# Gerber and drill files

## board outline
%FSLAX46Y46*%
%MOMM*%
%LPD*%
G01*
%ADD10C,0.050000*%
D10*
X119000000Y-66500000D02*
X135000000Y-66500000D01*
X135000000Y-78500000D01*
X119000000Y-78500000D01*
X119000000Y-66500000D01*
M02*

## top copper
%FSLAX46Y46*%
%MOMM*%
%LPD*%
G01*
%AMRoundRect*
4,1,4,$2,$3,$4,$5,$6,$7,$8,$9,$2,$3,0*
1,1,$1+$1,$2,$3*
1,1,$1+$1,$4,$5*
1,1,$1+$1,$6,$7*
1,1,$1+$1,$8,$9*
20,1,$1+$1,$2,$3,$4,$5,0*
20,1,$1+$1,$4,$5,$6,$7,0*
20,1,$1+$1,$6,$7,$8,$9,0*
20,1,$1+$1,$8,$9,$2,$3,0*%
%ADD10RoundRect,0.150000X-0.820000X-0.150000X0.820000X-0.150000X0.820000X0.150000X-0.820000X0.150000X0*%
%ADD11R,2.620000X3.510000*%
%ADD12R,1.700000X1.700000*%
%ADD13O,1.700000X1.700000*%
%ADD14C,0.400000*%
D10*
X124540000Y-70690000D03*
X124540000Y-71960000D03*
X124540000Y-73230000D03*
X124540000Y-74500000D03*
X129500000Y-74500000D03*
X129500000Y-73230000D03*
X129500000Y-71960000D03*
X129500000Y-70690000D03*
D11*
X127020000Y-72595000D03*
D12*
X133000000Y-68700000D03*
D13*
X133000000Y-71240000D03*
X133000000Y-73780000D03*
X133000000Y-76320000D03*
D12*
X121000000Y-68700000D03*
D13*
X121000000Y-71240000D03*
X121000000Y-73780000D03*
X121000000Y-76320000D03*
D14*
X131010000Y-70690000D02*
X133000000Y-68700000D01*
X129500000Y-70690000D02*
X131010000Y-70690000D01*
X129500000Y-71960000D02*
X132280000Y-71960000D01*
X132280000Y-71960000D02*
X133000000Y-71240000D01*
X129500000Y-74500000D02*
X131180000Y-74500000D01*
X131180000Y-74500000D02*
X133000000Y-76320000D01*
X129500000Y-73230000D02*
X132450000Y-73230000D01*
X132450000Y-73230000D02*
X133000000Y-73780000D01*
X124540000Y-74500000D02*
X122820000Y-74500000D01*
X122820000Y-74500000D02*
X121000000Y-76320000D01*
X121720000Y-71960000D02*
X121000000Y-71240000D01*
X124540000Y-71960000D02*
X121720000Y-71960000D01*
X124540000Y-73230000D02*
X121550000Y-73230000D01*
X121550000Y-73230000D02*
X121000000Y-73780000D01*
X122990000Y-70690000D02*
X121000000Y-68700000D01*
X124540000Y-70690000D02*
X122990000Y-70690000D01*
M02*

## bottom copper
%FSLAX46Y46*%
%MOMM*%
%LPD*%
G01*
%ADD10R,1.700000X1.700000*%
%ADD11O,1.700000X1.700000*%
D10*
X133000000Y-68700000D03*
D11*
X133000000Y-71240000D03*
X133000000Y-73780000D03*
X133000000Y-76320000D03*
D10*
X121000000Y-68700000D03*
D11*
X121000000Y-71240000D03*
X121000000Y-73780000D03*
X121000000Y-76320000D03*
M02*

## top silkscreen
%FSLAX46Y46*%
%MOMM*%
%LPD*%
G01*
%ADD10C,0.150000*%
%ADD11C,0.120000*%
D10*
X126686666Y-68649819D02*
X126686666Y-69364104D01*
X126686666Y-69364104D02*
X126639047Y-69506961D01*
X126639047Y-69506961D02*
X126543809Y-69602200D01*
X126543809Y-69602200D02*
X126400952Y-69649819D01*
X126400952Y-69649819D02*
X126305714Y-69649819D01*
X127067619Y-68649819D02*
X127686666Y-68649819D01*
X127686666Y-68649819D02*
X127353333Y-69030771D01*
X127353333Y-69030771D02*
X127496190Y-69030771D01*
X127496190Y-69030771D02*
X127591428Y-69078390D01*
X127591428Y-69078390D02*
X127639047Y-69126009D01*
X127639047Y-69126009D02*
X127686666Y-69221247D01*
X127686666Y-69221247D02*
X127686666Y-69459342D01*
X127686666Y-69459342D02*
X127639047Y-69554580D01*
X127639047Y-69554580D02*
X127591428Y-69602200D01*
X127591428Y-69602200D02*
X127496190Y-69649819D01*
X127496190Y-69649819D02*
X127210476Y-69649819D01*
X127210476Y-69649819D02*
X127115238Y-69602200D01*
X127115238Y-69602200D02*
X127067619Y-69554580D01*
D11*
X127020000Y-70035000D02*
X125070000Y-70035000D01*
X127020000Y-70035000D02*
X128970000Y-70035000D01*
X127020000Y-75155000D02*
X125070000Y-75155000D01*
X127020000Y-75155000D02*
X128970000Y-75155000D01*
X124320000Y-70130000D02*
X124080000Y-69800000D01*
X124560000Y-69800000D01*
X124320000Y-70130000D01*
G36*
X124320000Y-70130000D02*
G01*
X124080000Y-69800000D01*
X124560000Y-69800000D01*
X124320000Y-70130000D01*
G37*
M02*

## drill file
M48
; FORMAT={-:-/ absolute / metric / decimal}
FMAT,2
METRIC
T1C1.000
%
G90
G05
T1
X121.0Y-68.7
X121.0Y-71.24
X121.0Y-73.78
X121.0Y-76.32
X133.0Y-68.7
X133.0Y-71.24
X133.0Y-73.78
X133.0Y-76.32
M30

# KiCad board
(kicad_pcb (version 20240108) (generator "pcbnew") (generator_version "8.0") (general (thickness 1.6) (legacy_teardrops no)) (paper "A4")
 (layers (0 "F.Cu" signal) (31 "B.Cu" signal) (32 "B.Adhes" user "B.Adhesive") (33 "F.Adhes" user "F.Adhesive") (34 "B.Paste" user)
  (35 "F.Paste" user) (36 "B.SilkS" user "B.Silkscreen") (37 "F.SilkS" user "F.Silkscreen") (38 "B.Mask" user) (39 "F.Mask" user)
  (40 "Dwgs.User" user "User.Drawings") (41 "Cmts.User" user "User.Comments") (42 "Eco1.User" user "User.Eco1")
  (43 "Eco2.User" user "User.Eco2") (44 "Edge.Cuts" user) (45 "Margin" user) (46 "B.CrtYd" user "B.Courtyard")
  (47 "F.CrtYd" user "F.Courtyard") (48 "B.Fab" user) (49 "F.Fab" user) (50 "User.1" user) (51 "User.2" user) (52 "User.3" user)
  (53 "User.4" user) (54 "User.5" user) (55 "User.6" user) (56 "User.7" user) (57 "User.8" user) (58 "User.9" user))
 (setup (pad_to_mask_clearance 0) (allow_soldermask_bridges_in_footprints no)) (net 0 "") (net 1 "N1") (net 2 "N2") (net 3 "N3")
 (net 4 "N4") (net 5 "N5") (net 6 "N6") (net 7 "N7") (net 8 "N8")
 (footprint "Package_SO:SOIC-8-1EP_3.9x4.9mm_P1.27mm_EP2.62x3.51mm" (layer "F.Cu") (at 127.02 72.595)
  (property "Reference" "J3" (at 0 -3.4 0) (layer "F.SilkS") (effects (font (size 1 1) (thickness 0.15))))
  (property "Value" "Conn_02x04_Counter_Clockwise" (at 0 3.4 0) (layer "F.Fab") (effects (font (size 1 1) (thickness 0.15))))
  (fp_line (start 0 -2.56) (end -1.95 -2.56) (stroke (width 0.12) (type solid)) (layer "F.SilkS"))
  (fp_line (start 0 -2.56) (end 1.95 -2.56) (stroke (width 0.12) (type solid)) (layer "F.SilkS"))
  (fp_line (start 0 2.56) (end -1.95 2.56) (stroke (width 0.12) (type solid)) (layer "F.SilkS"))
  (fp_line (start 0 2.56) (end 1.95 2.56) (stroke (width 0.12) (type solid)) (layer "F.SilkS"))
  (fp_poly
   (pts (xy -2.7 -2.465) (xy -2.94 -2.795) (xy -2.46 -2.795) (xy -2.7 -2.465)) (stroke (width 0.12) (type solid)) (fill solid)
   (layer "F.SilkS"))
  (pad "" smd roundrect (at -0.655 -0.875) (size 1.06 1.41) (layers "F.Paste") (roundrect_rratio 0.235849))
  (pad "" smd roundrect (at -0.655 0.875) (size 1.06 1.41) (layers "F.Paste") (roundrect_rratio 0.235849))
  (pad "" smd roundrect (at 0.655 -0.875) (size 1.06 1.41) (layers "F.Paste") (roundrect_rratio 0.235849))
  (pad "" smd roundrect (at 0.655 0.875) (size 1.06 1.41) (layers "F.Paste") (roundrect_rratio 0.235849))
  (pad "1" smd roundrect (at -2.48 -1.905) (size 1.94 0.6) (layers "F.Cu" "F.Paste" "F.Mask") (roundrect_rratio 0.25) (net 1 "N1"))
  (pad "2" smd roundrect (at -2.48 -0.635) (size 1.94 0.6) (layers "F.Cu" "F.Paste" "F.Mask") (roundrect_rratio 0.25) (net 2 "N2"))
  (pad "3" smd roundrect (at -2.48 0.635) (size 1.94 0.6) (layers "F.Cu" "F.Paste" "F.Mask") (roundrect_rratio 0.25) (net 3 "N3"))
  (pad "4" smd roundrect (at -2.48 1.905) (size 1.94 0.6) (layers "F.Cu" "F.Paste" "F.Mask") (roundrect_rratio 0.25) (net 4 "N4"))
  (pad "5" smd roundrect (at 2.48 1.905) (size 1.94 0.6) (layers "F.Cu" "F.Paste" "F.Mask") (roundrect_rratio 0.25) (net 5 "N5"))
  (pad "6" smd roundrect (at 2.48 0.635) (size 1.94 0.6) (layers "F.Cu" "F.Paste" "F.Mask") (roundrect_rratio 0.25) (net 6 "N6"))
  (pad "7" smd roundrect (at 2.48 -0.635) (size 1.94 0.6) (layers "F.Cu" "F.Paste" "F.Mask") (roundrect_rratio 0.25) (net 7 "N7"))
  (pad "8" smd roundrect (at 2.48 -1.905) (size 1.94 0.6) (layers "F.Cu" "F.Paste" "F.Mask") (roundrect_rratio 0.25) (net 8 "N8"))
  (pad "9" smd rect (at 0 0) (size 2.62 3.51) (layers "F.Cu" "F.Mask") (zone_connect 2)))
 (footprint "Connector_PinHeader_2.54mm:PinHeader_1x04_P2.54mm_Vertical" (layer "B.Cu") (at 133 68.7 180)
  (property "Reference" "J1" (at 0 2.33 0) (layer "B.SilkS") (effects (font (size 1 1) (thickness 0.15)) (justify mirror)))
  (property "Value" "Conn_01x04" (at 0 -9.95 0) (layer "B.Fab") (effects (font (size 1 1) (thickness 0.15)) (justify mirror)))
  (pad "1" thru_hole rect (at 0 0 180) (size 1.7 1.7) (drill 1) (layers "*.Cu" "*.Mask") (remove_unused_layers no) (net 8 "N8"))
  (pad "2" thru_hole oval (at 0 -2.54 180) (size 1.7 1.7) (drill 1) (layers "*.Cu" "*.Mask") (remove_unused_layers no) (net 7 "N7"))
  (pad "3" thru_hole oval (at 0 -5.08 180) (size 1.7 1.7) (drill 1) (layers "*.Cu" "*.Mask") (remove_unused_layers no) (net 6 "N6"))
  (pad "4" thru_hole oval (at 0 -7.62 180) (size 1.7 1.7) (drill 1) (layers "*.Cu" "*.Mask") (remove_unused_layers no) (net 5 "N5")))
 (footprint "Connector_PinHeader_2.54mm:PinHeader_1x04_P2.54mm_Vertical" (layer "B.Cu") (at 121 68.7 180)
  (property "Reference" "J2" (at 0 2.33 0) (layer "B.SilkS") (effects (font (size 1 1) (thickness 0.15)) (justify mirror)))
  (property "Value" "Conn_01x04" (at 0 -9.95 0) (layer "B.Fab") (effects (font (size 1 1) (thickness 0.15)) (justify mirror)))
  (pad "1" thru_hole rect (at 0 0 180) (size 1.7 1.7) (drill 1) (layers "*.Cu" "*.Mask") (remove_unused_layers no) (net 1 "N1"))
  (pad "2" thru_hole oval (at 0 -2.54 180) (size 1.7 1.7) (drill 1) (layers "*.Cu" "*.Mask") (remove_unused_layers no) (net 2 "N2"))
  (pad "3" thru_hole oval (at 0 -5.08 180) (size 1.7 1.7) (drill 1) (layers "*.Cu" "*.Mask") (remove_unused_layers no) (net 3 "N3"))
  (pad "4" thru_hole oval (at 0 -7.62 180) (size 1.7 1.7) (drill 1) (layers "*.Cu" "*.Mask") (remove_unused_layers no) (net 4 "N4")))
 (gr_rect (start 119 66.5) (end 135 78.5) (stroke (width 0.05) (type default)) (fill none) (layer "Edge.Cuts"))
 (segment (start 131.01 70.69) (end 133 68.7) (width 0.4) (layer "F.Cu") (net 8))
 (segment (start 129.5 70.69) (end 131.01 70.69) (width 0.4) (layer "F.Cu") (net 8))
 (segment (start 129.5 71.96) (end 132.28 71.96) (width 0.4) (layer "F.Cu") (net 7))
 (segment (start 132.28 71.96) (end 133 71.24) (width 0.4) (layer "F.Cu") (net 7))
 (segment (start 129.5 74.5) (end 131.18 74.5) (width 0.4) (layer "F.Cu") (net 5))
 (segment (start 131.18 74.5) (end 133 76.32) (width 0.4) (layer "F.Cu") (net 5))
 (segment (start 129.5 73.23) (end 132.45 73.23) (width 0.4) (layer "F.Cu") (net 6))
 (segment (start 132.45 73.23) (end 133 73.78) (width 0.4) (layer "F.Cu") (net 6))
 (segment (start 124.54 74.5) (end 122.82 74.5) (width 0.4) (layer "F.Cu") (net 4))
 (segment (start 122.82 74.5) (end 121 76.32) (width 0.4) (layer "F.Cu") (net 4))
 (segment (start 121.72 71.96) (end 121 71.24) (width 0.4) (layer "F.Cu") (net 2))
 (segment (start 124.54 71.96) (end 121.72 71.96) (width 0.4) (layer "F.Cu") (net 2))
 (segment (start 124.54 73.23) (end 121.55 73.23) (width 0.4) (layer "F.Cu") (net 3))
 (segment (start 121.55 73.23) (end 121 73.78) (width 0.4) (layer "F.Cu") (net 3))
 (segment (start 122.99 70.69) (end 121 68.7) (width 0.4) (layer "F.Cu") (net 1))
 (segment (start 124.54 70.69) (end 122.99 70.69) (width 0.4) (layer "F.Cu") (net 1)))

